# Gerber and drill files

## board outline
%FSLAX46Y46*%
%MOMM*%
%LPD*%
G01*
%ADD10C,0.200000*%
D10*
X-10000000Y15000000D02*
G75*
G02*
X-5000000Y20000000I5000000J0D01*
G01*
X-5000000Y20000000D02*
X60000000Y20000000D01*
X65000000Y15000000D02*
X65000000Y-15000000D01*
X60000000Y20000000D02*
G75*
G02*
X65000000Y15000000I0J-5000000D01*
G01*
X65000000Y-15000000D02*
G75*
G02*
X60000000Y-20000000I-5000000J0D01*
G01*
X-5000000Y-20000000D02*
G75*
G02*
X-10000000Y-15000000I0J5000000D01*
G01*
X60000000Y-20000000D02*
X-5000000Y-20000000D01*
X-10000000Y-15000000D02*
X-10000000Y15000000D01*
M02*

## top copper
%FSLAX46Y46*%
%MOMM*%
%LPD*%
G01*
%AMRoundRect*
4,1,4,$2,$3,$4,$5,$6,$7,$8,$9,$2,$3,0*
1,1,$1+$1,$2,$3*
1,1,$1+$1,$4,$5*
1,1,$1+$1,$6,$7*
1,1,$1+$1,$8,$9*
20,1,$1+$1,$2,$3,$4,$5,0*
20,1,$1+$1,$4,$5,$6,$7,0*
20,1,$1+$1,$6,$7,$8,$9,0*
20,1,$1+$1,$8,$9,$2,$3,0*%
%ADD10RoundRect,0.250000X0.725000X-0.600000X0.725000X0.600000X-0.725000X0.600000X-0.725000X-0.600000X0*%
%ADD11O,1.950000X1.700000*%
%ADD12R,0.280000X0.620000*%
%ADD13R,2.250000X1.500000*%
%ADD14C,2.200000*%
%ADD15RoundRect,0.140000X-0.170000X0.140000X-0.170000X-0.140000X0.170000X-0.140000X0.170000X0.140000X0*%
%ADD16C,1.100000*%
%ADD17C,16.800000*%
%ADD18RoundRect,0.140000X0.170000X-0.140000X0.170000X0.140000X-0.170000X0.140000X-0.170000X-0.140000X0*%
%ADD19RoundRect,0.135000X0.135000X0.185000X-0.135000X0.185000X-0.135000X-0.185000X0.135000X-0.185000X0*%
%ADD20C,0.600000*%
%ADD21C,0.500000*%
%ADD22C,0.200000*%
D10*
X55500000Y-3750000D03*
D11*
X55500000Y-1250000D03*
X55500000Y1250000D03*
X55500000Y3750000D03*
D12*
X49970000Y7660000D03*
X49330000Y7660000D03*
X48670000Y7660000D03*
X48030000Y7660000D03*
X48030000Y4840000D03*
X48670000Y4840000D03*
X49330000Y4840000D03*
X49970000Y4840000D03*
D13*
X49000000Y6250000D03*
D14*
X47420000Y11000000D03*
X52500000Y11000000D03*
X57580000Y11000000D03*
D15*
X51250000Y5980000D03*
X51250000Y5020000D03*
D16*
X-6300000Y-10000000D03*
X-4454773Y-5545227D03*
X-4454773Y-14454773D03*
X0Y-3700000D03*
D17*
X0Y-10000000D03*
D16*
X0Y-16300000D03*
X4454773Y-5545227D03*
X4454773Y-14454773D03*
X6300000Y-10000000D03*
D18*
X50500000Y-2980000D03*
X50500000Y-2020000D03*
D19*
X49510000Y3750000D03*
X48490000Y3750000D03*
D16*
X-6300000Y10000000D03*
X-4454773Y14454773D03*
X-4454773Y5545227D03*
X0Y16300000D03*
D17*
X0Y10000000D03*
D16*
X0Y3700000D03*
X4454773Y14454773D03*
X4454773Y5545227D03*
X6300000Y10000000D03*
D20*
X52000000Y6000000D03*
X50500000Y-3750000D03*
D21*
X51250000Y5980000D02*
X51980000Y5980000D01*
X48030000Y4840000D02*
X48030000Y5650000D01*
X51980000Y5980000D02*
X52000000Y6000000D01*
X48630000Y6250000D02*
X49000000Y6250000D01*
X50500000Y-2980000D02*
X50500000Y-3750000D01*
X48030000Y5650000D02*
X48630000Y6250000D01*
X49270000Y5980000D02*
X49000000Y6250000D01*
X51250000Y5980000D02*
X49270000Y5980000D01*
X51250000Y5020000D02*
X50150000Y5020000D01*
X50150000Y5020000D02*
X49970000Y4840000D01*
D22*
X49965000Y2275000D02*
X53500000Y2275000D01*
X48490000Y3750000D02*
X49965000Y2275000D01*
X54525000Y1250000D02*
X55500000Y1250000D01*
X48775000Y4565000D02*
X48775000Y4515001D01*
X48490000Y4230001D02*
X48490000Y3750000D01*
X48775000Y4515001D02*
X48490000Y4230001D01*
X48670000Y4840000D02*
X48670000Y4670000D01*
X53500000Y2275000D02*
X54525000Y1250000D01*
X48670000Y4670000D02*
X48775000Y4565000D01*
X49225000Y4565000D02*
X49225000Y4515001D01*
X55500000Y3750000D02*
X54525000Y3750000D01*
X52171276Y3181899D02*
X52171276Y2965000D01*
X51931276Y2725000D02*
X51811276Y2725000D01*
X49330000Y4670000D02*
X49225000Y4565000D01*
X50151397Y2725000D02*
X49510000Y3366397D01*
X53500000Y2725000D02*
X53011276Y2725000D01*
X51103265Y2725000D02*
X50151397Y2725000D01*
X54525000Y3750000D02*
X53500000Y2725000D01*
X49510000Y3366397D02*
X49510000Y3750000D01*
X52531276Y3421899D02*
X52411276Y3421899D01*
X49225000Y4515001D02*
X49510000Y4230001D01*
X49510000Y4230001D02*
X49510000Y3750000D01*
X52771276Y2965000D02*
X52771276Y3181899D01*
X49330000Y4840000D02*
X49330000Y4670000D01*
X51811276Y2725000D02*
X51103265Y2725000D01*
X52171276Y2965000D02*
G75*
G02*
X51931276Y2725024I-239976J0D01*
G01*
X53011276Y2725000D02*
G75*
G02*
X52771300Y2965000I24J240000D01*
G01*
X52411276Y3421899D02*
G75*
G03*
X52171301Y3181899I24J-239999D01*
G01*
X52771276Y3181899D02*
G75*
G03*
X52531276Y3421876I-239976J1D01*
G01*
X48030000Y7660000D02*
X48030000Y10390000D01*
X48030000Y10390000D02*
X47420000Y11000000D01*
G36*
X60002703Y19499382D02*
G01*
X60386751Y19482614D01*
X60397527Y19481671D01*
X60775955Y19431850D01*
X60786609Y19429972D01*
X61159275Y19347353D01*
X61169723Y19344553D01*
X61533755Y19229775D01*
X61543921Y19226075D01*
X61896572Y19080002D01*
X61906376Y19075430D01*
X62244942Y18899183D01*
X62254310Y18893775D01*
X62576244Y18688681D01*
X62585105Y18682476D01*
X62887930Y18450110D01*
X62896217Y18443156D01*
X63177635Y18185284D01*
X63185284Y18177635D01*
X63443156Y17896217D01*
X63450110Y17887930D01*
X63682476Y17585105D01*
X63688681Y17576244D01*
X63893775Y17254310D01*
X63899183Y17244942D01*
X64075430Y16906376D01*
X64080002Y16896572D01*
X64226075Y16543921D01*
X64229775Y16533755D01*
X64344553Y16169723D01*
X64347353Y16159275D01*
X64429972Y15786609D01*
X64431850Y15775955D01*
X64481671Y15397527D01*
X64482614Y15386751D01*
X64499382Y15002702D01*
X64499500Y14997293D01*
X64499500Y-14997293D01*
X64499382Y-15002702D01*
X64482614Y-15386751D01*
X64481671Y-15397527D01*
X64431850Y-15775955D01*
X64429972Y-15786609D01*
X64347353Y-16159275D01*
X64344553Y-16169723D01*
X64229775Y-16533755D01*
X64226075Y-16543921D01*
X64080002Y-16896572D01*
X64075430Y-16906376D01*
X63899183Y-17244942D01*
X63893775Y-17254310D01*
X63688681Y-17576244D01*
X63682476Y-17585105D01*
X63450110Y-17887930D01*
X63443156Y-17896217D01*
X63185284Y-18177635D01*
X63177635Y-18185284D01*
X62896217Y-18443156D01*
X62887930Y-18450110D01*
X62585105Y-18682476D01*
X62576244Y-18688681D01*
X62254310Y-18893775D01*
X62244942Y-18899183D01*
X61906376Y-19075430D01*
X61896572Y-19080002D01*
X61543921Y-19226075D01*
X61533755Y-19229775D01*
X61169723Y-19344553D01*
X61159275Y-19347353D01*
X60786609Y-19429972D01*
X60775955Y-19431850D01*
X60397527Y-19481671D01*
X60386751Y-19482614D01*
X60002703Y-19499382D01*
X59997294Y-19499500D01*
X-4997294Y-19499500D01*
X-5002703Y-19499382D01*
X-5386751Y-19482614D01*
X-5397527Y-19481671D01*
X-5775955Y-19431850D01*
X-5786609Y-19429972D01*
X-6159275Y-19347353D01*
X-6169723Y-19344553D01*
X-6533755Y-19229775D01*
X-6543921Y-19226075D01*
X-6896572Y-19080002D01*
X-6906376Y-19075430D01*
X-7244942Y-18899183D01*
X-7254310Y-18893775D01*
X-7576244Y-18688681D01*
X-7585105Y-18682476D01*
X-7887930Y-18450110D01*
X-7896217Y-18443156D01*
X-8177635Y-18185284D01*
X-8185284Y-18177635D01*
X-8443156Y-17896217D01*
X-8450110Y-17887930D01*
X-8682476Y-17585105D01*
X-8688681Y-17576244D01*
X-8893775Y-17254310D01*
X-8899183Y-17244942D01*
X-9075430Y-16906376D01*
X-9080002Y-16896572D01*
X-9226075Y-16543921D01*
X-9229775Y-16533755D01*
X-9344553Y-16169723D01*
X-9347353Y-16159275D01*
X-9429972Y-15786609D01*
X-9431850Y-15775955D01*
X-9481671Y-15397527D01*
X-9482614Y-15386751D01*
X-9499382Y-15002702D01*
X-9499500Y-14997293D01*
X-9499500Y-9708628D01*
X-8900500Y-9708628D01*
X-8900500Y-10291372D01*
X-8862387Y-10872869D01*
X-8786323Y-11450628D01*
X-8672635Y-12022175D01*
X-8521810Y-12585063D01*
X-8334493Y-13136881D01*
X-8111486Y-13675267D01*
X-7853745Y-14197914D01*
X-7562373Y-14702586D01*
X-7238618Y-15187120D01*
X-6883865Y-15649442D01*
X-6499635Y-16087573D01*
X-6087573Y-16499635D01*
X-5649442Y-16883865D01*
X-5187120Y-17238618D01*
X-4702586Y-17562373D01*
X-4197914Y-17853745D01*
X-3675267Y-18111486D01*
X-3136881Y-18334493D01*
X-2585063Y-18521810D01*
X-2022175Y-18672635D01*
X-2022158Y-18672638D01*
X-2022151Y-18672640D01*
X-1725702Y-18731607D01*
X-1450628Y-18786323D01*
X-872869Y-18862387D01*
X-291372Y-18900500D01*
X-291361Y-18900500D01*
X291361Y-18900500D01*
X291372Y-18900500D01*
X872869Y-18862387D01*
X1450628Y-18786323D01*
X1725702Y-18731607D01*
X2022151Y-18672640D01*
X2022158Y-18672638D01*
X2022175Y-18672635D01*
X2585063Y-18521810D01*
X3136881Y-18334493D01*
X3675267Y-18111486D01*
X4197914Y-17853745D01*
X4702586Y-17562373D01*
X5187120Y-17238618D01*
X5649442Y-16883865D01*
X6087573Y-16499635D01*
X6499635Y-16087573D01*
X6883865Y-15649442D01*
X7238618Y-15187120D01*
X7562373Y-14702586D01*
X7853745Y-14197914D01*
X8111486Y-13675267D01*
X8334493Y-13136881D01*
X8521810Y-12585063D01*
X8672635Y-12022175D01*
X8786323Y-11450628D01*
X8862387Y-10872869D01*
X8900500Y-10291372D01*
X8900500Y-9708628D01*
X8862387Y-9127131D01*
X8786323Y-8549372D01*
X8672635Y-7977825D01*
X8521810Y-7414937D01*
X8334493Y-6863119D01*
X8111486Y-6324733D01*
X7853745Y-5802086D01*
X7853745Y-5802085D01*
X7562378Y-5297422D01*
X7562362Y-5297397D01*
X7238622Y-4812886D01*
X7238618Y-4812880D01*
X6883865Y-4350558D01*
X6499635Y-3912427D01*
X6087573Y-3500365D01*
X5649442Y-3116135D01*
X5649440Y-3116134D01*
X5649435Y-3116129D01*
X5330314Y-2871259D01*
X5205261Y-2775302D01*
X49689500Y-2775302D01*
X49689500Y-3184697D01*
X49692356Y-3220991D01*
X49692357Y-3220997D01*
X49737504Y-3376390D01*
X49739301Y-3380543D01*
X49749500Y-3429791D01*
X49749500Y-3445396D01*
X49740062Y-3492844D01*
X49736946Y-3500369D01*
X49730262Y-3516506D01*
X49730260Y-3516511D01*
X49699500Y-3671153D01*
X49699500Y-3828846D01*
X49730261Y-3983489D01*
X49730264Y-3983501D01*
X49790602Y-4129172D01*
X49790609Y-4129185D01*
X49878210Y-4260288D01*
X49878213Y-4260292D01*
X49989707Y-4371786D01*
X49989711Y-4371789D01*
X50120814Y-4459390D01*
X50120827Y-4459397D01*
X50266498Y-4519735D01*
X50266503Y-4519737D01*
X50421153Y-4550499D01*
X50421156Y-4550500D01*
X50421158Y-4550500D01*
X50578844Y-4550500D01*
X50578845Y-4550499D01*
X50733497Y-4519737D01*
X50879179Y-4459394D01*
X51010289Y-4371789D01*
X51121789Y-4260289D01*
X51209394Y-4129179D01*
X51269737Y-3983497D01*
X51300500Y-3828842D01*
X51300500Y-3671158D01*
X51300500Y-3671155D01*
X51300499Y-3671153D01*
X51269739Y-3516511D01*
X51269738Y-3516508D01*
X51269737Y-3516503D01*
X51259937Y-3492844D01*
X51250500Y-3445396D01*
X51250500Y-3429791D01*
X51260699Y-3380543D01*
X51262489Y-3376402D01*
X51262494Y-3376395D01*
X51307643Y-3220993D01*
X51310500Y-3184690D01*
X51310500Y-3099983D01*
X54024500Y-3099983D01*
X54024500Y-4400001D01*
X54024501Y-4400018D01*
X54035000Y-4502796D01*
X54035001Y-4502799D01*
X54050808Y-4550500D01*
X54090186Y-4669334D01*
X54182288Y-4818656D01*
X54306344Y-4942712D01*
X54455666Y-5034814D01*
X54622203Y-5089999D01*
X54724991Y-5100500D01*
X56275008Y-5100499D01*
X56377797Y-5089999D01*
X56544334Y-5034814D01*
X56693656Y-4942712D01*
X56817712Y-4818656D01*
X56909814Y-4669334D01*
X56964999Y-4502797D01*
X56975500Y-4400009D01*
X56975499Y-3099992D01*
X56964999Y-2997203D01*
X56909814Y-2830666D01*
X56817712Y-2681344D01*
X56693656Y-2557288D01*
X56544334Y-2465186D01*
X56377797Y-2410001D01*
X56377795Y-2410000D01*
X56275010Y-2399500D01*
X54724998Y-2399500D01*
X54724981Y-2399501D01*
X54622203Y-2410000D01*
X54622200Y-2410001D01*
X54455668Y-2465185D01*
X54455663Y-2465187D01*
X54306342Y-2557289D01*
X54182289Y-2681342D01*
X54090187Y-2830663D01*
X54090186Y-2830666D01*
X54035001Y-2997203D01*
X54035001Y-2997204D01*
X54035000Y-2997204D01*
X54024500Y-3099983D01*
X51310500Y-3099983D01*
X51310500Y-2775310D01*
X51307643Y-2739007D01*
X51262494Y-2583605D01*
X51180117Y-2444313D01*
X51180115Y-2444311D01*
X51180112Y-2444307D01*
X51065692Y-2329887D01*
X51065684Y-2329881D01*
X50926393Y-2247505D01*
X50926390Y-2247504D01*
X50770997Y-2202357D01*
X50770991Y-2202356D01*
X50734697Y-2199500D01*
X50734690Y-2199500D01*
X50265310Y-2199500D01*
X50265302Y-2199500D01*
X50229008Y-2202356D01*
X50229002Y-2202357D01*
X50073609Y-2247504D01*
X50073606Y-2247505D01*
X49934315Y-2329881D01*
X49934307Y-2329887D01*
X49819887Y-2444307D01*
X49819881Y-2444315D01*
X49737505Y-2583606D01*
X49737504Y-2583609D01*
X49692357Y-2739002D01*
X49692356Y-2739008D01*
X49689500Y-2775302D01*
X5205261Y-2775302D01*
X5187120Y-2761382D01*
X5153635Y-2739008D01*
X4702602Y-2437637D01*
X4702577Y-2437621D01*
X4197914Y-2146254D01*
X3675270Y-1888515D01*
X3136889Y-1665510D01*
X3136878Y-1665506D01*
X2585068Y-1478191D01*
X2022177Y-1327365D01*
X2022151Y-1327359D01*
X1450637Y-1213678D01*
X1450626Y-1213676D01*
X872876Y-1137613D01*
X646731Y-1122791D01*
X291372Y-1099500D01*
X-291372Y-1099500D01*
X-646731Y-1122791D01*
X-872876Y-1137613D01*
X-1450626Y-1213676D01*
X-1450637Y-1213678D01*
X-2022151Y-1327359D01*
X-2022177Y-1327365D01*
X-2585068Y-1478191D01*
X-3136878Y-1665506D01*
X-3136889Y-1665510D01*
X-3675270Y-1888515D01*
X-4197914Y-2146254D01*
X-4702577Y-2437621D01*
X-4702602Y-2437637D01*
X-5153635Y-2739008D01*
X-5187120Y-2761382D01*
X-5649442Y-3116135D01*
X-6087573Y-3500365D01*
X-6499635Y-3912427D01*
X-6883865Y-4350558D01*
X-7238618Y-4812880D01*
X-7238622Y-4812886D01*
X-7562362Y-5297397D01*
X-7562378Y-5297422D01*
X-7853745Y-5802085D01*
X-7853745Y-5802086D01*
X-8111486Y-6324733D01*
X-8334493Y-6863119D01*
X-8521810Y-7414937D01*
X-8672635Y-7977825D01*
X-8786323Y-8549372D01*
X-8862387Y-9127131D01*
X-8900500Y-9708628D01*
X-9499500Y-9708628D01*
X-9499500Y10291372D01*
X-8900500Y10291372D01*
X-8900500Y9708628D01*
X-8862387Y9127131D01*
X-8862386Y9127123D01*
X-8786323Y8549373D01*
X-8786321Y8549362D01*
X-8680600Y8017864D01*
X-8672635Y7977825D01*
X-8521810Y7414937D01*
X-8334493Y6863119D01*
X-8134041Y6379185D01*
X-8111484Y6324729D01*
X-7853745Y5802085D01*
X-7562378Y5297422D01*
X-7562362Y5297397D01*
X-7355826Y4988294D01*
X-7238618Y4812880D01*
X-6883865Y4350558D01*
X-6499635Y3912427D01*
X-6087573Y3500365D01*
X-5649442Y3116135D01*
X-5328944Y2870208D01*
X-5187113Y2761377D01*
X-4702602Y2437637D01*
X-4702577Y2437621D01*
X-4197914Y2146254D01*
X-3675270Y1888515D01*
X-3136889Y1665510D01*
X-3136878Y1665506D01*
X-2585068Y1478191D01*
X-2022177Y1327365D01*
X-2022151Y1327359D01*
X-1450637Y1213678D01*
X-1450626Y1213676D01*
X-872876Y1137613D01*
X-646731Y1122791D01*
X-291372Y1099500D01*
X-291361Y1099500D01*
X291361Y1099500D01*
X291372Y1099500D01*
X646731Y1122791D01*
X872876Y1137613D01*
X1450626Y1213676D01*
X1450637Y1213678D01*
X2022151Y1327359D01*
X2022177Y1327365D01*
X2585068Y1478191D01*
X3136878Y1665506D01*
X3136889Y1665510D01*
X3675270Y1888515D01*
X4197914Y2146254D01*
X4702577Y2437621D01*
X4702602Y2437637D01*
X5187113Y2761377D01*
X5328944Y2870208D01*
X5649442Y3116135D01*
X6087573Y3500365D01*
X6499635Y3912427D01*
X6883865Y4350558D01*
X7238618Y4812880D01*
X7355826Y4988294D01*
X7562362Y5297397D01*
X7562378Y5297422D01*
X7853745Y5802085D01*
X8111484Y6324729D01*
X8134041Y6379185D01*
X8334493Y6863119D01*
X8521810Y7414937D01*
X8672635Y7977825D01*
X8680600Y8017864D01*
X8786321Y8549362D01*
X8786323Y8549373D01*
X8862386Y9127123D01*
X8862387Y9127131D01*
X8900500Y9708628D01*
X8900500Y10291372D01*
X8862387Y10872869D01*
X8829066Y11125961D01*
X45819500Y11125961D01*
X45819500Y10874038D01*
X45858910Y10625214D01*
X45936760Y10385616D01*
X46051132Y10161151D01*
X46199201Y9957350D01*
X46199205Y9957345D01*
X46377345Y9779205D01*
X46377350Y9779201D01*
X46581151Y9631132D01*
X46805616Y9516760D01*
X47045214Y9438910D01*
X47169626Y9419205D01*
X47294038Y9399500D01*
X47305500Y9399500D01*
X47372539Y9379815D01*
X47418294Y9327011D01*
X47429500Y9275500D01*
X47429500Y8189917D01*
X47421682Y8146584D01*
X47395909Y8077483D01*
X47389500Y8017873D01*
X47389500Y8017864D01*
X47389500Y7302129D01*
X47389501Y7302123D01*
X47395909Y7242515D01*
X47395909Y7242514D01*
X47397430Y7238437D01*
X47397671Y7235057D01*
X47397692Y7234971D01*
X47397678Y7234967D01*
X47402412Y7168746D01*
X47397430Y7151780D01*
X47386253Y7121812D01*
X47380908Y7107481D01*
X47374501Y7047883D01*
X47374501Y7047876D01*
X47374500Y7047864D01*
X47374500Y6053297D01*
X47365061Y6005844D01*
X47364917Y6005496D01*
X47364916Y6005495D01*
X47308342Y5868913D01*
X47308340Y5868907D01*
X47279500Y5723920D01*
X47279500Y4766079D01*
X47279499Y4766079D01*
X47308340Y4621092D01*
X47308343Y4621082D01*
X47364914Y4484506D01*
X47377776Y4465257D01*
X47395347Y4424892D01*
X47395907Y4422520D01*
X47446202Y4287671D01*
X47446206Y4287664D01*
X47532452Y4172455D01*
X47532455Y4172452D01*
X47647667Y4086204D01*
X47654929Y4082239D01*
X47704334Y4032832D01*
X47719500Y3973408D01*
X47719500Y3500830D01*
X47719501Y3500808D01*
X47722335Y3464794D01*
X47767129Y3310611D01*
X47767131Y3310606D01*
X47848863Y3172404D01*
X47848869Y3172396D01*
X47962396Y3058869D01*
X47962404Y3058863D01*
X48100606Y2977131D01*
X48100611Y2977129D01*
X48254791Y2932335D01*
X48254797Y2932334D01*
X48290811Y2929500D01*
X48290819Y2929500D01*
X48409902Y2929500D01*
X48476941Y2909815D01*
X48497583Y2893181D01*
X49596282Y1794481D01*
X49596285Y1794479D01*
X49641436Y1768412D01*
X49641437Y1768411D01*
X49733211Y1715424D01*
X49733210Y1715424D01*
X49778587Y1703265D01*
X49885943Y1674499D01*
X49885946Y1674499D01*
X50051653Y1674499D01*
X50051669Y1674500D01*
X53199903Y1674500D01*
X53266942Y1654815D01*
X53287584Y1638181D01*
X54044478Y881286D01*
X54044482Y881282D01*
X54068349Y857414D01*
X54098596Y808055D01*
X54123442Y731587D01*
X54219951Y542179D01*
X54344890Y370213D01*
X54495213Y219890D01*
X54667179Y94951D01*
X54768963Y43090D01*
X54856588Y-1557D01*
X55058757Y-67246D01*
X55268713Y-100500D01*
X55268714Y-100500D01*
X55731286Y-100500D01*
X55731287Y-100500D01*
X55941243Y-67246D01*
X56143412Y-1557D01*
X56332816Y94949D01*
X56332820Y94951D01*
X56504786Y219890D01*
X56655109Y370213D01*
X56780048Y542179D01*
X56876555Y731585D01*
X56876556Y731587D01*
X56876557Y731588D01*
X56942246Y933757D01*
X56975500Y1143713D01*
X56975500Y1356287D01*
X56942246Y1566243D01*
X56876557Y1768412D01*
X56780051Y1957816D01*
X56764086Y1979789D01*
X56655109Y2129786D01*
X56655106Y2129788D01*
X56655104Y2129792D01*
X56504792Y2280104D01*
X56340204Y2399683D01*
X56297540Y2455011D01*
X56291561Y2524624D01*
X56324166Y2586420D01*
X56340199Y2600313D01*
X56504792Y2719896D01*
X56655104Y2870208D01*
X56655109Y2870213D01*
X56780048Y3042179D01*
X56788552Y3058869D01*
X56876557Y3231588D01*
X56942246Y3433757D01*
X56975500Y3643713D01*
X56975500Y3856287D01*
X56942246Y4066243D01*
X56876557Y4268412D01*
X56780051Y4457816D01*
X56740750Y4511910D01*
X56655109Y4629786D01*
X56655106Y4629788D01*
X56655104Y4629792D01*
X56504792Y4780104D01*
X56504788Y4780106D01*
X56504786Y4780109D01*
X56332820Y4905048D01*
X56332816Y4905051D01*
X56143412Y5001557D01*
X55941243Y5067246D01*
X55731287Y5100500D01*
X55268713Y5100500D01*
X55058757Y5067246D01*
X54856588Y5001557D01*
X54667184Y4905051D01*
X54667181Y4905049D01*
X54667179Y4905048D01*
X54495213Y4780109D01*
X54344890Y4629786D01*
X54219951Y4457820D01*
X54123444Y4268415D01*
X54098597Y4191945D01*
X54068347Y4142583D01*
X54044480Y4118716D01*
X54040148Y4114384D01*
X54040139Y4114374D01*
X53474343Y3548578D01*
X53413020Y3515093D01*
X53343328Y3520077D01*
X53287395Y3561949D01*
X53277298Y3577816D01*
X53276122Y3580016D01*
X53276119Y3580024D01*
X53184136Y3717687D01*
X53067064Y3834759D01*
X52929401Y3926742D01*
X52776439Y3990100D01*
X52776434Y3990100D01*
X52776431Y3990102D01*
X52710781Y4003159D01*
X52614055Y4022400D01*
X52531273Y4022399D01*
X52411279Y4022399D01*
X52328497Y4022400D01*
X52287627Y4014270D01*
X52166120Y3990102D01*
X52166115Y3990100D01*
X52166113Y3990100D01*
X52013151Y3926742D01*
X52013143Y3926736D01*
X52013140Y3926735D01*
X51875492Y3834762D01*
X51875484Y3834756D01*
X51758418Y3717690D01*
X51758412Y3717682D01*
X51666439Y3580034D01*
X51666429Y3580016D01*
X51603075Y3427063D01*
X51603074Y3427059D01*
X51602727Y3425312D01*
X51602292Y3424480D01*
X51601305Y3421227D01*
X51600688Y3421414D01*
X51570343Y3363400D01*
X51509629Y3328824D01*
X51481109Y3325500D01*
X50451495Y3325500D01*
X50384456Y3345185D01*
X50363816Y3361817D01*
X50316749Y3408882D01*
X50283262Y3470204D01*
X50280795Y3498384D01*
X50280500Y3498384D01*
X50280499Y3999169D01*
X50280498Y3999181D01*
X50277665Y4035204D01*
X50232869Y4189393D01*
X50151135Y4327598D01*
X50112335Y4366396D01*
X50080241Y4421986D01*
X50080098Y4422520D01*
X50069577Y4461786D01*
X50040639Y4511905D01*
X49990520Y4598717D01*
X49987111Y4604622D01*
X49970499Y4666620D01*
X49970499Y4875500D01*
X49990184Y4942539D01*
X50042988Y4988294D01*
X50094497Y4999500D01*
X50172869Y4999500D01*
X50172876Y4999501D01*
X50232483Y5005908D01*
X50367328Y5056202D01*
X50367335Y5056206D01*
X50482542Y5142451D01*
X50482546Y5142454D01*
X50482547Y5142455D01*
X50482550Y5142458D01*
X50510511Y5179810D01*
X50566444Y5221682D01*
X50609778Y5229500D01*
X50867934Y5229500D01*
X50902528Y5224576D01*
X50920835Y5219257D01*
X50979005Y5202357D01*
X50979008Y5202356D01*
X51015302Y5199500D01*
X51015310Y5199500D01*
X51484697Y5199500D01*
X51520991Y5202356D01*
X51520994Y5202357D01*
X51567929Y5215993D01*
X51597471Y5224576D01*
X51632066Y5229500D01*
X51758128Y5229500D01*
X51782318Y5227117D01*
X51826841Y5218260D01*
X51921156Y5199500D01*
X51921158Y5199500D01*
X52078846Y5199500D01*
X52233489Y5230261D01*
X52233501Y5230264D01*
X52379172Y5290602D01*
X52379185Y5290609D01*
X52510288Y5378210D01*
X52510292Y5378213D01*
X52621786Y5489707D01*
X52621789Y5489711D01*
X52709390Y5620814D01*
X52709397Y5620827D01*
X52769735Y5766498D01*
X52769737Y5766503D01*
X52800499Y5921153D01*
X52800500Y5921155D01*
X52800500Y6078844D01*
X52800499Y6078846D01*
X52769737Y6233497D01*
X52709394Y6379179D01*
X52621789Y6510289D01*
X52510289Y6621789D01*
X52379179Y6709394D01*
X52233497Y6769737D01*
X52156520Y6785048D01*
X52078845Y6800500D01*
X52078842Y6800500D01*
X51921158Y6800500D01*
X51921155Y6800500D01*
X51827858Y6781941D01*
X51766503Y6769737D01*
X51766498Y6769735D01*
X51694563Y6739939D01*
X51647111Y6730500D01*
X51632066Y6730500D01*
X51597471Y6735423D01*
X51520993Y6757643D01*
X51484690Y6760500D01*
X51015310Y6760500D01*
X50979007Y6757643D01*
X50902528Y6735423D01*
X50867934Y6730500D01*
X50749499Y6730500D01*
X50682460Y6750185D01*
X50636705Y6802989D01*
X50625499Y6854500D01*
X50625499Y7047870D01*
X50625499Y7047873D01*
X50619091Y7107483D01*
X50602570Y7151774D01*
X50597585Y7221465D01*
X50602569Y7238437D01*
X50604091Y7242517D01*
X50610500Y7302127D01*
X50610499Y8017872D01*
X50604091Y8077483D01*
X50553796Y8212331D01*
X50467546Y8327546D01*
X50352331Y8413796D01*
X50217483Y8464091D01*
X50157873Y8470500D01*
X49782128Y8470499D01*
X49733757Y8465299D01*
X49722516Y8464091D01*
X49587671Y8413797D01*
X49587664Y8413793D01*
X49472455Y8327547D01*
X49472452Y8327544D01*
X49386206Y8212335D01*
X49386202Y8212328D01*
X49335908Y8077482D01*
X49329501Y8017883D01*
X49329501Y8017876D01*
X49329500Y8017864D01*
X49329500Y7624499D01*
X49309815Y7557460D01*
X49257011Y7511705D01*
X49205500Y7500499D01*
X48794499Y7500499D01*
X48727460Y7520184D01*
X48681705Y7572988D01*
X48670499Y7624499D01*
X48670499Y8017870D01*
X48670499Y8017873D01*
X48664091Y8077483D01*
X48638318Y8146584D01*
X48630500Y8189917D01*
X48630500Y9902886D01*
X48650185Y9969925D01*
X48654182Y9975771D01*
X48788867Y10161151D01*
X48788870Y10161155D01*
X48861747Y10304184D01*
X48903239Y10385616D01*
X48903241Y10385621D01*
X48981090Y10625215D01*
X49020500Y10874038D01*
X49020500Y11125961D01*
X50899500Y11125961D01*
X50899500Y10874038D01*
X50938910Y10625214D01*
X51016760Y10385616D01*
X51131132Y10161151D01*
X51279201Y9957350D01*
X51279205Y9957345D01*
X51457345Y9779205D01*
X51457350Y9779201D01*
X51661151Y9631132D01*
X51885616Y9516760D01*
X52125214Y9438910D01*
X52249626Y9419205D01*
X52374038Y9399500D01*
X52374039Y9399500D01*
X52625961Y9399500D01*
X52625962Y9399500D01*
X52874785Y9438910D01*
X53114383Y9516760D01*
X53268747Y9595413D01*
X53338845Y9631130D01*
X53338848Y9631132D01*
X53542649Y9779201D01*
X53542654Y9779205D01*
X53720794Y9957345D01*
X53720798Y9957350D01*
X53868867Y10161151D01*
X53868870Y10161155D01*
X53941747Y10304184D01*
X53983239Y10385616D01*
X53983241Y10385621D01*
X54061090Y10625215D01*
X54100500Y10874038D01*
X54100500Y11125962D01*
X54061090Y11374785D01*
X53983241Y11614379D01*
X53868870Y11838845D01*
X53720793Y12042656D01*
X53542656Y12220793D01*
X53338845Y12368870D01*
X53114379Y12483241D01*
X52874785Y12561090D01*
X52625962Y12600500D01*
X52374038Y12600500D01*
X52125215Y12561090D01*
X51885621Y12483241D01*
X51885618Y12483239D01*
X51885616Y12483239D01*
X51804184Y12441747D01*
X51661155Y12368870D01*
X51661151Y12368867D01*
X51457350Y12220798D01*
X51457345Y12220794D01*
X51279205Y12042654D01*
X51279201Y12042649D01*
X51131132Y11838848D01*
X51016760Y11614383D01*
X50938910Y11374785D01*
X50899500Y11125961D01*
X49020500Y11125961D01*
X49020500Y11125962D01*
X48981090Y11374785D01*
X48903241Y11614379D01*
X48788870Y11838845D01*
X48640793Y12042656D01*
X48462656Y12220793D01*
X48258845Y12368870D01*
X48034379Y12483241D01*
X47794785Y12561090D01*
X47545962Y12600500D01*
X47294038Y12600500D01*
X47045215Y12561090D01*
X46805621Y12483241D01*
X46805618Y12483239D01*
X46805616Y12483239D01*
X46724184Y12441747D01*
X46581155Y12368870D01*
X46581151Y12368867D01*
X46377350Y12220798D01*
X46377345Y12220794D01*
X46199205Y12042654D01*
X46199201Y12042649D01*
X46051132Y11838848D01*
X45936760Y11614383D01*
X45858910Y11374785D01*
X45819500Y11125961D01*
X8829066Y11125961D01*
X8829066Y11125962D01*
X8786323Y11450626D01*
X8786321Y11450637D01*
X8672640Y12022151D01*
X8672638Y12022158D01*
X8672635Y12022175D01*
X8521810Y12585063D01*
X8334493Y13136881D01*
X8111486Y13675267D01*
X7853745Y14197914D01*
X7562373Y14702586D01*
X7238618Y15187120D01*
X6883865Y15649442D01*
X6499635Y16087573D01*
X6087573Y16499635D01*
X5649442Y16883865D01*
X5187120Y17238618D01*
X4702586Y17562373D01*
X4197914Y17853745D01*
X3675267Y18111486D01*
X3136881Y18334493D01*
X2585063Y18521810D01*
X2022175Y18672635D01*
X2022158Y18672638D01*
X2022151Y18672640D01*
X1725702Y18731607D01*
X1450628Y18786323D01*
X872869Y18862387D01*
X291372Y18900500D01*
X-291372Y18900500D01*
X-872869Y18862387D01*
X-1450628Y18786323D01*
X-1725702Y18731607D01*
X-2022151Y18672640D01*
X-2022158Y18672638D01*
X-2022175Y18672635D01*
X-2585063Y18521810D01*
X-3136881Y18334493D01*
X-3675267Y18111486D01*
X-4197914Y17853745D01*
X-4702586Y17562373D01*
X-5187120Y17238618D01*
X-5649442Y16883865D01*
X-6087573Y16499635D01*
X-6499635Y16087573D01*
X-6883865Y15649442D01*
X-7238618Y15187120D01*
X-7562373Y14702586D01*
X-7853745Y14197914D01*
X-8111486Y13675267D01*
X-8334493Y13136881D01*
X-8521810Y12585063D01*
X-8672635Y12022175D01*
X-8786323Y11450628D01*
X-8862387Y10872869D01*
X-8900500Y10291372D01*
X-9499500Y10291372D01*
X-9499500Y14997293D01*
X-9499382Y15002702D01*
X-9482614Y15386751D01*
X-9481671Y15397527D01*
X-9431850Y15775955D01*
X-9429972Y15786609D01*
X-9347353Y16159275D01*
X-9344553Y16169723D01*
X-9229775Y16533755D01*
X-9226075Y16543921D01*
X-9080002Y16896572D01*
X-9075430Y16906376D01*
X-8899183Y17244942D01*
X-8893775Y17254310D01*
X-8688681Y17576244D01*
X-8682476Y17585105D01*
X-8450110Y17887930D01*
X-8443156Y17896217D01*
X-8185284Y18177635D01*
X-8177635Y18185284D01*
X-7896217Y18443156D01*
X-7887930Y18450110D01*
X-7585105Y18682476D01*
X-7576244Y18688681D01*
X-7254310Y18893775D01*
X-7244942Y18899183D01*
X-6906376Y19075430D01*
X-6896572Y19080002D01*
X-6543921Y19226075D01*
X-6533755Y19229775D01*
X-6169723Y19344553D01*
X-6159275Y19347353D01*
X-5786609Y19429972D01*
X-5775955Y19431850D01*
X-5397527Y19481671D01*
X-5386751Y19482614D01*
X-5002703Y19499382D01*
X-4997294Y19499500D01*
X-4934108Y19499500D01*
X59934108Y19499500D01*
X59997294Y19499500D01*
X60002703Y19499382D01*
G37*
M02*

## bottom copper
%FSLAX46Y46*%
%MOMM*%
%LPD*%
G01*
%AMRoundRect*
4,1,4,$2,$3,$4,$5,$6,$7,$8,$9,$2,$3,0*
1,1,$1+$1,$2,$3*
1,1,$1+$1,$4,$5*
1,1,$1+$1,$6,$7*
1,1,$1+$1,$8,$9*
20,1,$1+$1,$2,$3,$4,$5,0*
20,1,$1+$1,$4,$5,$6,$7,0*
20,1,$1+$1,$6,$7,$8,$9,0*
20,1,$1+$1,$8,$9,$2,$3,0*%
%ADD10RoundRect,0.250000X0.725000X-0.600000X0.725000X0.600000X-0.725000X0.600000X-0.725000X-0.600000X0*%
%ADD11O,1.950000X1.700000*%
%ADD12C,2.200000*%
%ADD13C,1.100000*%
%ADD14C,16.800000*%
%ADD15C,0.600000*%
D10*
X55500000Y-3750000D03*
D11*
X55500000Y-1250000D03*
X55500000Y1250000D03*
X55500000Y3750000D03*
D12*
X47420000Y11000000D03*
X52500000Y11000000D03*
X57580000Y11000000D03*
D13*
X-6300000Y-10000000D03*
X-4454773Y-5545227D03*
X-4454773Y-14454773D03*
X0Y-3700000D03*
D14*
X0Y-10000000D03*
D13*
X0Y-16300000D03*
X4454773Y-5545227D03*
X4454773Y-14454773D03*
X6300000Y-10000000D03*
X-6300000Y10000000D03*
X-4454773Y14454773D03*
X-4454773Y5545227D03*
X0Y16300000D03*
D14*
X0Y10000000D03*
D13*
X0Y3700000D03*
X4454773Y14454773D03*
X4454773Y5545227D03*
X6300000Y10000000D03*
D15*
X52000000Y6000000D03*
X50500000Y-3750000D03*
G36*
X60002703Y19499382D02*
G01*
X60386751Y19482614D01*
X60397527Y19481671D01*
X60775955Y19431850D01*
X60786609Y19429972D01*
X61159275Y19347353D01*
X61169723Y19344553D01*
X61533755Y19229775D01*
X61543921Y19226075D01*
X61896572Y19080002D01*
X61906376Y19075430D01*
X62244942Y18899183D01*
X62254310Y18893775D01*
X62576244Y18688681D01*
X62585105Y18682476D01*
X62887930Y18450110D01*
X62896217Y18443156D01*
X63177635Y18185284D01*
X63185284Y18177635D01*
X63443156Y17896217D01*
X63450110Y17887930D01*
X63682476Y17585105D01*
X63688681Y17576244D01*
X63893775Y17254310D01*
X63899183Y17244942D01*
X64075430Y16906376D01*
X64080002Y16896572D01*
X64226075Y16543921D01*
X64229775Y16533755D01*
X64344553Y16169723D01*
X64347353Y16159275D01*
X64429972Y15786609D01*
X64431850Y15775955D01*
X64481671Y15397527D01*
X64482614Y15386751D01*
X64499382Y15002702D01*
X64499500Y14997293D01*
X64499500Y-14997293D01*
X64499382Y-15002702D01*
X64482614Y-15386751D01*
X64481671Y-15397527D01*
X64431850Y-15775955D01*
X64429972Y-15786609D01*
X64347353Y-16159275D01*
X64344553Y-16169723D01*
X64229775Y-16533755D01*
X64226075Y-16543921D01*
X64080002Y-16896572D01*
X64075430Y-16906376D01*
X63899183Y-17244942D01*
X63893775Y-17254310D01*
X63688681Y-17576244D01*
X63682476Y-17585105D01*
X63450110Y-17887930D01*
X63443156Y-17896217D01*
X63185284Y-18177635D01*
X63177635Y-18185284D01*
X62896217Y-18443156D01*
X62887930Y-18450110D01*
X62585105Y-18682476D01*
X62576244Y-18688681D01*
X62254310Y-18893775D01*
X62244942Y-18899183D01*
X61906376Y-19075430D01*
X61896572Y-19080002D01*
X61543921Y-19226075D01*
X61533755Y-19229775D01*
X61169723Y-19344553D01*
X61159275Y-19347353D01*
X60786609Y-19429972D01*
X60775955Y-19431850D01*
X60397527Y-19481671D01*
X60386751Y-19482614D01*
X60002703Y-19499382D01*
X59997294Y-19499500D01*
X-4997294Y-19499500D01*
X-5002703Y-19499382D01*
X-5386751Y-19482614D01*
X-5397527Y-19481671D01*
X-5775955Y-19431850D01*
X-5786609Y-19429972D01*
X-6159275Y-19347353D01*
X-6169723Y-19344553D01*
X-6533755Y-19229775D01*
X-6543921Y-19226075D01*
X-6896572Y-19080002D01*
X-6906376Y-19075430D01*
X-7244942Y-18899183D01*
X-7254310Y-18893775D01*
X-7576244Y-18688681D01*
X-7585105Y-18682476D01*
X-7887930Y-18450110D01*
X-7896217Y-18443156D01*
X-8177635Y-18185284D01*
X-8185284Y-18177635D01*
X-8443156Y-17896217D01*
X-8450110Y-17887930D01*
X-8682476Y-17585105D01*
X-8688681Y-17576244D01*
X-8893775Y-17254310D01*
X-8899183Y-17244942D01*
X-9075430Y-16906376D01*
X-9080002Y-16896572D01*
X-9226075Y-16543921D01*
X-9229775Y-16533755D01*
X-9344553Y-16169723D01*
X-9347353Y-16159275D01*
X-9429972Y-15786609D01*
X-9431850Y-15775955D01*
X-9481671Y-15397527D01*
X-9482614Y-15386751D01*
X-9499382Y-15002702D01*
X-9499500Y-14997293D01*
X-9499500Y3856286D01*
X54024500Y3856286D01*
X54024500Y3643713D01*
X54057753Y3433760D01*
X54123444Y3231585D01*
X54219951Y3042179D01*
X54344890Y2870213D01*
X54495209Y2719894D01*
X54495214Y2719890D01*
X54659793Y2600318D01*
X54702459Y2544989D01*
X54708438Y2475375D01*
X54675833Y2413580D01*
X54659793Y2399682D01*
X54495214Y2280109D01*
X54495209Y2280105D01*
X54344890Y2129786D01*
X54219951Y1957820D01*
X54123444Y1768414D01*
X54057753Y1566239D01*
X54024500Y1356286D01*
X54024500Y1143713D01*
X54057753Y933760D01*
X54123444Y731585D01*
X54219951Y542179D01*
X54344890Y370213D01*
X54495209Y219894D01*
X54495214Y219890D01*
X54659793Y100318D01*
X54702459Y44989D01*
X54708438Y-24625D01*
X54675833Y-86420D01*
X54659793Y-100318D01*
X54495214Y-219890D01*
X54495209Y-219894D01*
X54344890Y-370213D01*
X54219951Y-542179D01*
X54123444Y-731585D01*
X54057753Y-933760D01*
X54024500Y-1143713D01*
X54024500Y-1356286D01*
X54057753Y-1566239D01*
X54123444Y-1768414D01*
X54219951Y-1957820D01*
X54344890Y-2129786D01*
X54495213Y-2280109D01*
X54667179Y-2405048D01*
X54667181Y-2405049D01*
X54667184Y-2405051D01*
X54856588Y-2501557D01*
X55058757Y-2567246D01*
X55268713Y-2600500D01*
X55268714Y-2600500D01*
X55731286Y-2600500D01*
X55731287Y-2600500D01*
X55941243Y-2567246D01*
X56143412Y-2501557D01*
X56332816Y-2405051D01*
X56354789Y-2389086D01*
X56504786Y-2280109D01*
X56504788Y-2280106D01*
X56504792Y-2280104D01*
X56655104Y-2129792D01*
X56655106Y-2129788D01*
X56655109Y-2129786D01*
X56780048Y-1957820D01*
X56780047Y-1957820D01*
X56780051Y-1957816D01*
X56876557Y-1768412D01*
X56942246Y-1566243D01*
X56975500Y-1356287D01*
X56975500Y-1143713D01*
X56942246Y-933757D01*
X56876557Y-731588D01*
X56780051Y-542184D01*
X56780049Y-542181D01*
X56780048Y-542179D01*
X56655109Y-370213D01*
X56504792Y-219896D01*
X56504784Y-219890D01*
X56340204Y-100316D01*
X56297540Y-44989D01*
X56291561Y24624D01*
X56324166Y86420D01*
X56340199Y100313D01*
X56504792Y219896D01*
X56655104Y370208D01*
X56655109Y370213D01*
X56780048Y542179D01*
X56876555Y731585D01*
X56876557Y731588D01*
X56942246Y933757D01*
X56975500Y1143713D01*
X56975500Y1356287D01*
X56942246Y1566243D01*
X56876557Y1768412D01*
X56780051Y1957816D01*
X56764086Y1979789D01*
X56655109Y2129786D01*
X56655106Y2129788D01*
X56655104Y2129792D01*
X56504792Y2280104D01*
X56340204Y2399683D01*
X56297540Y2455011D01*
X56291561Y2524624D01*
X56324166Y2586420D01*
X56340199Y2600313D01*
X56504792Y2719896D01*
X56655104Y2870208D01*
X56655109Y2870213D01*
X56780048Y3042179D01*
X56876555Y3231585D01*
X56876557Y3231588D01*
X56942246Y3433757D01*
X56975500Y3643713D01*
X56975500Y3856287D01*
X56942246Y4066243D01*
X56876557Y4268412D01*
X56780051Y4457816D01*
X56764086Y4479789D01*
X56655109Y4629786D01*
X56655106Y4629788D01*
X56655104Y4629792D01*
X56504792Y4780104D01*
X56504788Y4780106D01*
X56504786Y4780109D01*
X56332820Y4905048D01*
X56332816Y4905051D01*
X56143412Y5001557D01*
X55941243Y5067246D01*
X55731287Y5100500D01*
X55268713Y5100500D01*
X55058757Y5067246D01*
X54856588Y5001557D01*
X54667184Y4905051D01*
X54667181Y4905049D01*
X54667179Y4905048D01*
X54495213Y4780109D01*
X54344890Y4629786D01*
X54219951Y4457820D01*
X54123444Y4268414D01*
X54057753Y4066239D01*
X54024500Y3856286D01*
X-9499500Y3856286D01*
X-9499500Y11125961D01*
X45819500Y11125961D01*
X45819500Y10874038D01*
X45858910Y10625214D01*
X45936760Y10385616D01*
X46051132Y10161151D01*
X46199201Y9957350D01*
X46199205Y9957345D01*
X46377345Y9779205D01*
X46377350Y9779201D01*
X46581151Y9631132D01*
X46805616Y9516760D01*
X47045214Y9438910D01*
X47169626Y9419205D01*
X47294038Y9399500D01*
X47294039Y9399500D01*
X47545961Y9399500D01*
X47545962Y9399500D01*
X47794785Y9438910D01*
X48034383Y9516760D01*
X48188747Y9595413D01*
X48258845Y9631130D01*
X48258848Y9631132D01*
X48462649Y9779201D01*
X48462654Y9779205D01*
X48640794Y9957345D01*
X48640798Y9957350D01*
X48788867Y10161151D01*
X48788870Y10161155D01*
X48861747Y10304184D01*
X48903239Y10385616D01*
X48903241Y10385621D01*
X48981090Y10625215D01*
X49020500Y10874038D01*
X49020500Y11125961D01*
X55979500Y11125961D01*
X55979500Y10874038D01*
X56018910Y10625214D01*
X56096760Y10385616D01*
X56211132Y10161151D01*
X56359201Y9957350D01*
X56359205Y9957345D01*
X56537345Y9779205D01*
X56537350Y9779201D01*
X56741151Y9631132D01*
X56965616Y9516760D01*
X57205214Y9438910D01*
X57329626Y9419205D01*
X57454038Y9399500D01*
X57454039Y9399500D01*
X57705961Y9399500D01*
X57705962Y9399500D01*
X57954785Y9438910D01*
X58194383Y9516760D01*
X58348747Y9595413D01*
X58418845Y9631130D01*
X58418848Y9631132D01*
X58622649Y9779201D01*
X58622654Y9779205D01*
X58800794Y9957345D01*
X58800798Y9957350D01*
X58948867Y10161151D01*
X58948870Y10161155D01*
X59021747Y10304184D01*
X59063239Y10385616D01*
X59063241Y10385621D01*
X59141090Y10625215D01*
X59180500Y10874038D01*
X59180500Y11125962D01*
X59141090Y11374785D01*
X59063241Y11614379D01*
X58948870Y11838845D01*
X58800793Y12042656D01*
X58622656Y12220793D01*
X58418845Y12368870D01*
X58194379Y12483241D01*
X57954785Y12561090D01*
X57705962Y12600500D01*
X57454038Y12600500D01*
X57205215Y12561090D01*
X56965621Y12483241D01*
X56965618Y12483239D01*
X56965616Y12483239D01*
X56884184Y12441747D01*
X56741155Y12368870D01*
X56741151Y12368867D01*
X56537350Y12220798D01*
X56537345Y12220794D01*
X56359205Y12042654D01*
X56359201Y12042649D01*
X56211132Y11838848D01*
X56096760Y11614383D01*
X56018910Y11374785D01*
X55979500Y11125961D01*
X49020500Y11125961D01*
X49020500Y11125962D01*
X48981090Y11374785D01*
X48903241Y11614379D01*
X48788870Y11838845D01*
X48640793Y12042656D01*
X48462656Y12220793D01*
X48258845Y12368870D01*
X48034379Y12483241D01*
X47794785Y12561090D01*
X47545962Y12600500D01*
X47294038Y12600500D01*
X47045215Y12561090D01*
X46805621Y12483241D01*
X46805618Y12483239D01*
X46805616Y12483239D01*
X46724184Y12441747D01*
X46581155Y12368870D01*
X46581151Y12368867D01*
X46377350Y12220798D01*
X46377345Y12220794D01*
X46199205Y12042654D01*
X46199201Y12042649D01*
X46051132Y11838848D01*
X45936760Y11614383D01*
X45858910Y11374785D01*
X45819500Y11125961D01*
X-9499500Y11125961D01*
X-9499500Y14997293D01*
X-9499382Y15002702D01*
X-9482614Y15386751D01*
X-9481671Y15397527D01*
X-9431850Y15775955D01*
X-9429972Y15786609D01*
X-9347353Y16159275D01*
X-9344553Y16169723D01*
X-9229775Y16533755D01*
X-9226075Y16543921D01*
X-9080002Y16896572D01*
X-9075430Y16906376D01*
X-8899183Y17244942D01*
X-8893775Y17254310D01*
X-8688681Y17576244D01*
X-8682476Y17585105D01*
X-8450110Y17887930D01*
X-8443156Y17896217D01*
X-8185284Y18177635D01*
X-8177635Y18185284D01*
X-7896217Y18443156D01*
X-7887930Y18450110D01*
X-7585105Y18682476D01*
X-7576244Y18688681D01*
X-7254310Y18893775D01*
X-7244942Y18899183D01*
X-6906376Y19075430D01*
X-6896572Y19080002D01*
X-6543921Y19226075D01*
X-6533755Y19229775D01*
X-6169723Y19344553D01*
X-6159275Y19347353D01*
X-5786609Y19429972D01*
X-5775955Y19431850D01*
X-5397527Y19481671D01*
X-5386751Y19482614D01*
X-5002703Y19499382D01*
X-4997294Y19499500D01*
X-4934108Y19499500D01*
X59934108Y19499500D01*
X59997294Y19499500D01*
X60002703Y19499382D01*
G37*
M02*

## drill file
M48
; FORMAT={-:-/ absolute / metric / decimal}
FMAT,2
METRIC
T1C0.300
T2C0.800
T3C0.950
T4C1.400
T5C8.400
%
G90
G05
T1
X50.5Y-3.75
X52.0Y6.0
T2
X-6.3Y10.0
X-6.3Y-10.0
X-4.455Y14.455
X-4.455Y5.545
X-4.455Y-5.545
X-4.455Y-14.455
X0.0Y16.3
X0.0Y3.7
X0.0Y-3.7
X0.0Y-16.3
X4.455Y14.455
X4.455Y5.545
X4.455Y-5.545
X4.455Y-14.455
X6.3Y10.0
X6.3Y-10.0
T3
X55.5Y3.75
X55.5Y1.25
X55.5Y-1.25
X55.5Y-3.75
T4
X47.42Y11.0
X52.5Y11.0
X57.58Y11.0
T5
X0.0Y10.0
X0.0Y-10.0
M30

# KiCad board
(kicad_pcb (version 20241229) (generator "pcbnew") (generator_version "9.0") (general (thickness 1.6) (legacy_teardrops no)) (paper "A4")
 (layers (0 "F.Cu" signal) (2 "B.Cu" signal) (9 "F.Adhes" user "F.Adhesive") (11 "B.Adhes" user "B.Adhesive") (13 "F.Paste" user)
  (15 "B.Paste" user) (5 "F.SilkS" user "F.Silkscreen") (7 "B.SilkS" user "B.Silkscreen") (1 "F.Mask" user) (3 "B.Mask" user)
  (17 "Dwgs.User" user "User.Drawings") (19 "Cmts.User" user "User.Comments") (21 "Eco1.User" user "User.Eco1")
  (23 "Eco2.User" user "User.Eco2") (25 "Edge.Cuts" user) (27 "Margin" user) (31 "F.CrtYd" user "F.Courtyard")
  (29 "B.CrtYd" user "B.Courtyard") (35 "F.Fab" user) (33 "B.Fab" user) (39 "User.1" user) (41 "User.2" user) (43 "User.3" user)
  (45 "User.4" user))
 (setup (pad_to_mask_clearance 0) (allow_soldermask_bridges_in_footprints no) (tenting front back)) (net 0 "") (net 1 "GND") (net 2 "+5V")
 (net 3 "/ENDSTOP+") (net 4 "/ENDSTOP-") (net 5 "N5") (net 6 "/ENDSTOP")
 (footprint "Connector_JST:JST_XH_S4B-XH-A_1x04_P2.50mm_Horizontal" (layer "F.Cu") (at 55.5 3.75 90)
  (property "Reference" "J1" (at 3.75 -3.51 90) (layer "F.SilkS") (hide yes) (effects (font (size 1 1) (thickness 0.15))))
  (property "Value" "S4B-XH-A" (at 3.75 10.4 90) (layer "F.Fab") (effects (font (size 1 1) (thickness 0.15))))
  (pad "1" thru_hole roundrect (at 0 0 90) (size 1.7 1.95) (drill 0.95) (layers "*.Cu" "*.Mask") (remove_unused_layers no)
   (roundrect_rratio 0.147059) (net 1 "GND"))
  (pad "2" thru_hole oval (at 2.5 0 90) (size 1.7 1.95) (drill 0.95) (layers "*.Cu" "*.Mask") (remove_unused_layers no) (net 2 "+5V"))
  (pad "3" thru_hole oval (at 5 0 90) (size 1.7 1.95) (drill 0.95) (layers "*.Cu" "*.Mask") (remove_unused_layers no) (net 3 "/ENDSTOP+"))
  (pad "4" thru_hole oval (at 7.5 0 90) (size 1.7 1.95) (drill 0.95) (layers "*.Cu" "*.Mask") (remove_unused_layers no) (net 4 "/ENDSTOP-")))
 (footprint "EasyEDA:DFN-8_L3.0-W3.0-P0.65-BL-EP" (layer "F.Cu") (at 49 -6.25 180)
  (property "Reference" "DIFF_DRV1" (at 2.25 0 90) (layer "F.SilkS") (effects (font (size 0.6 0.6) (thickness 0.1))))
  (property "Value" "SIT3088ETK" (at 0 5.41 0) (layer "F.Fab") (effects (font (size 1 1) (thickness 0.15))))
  (pad "1" smd rect (at -0.97 1.41 180) (size 0.28 0.62) (layers "F.Cu" "F.Mask" "F.Paste") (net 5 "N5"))
  (pad "2" smd rect (at -0.33 1.41 180) (size 0.28 0.62) (layers "F.Cu" "F.Mask" "F.Paste") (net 2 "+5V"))
  (pad "3" smd rect (at 0.33 1.41 180) (size 0.28 0.62) (layers "F.Cu" "F.Mask" "F.Paste") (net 2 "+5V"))
  (pad "4" smd rect (at 0.97 1.41 180) (size 0.28 0.62) (layers "F.Cu" "F.Mask" "F.Paste") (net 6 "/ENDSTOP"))
  (pad "5" smd rect (at 0.97 -1.41 180) (size 0.28 0.62) (layers "F.Cu" "F.Mask" "F.Paste") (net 1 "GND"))
  (pad "6" smd rect (at 0.33 -1.41 180) (size 0.28 0.62) (layers "F.Cu" "F.Mask" "F.Paste") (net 3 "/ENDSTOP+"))
  (pad "7" smd rect (at -0.33 -1.41 180) (size 0.28 0.62) (layers "F.Cu" "F.Mask" "F.Paste") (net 4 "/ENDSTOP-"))
  (pad "8" smd rect (at -0.97 -1.41 180) (size 0.28 0.62) (layers "F.Cu" "F.Mask" "F.Paste") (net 2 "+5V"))
  (pad "9" smd rect (at 0 0 180) (size 2.25 1.5) (layers "F.Cu" "F.Mask" "F.Paste") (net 1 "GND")))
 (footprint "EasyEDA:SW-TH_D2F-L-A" (layer "F.Cu") (at 52.5 -11)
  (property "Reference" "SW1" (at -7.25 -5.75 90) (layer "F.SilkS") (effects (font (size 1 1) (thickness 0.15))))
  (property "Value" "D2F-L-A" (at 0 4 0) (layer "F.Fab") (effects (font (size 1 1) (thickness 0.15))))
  (pad "1" thru_hole circle (at -5.08 0) (size 2.2 2.2) (drill 1.399997) (layers "*.Cu" "*.Mask") (remove_unused_layers no)
   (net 6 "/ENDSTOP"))
  (pad "2" thru_hole circle (at 0 0) (size 2.2 2.2) (drill 1.399997) (layers "*.Cu" "*.Mask") (remove_unused_layers no) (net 1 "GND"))
  (pad "3" thru_hole circle (at 5.08 0) (size 2.2 2.2) (drill 1.399997) (layers "*.Cu" "*.Mask") (remove_unused_layers no) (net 2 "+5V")))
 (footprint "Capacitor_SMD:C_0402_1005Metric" (layer "F.Cu") (at 51.25 -5.5 -90)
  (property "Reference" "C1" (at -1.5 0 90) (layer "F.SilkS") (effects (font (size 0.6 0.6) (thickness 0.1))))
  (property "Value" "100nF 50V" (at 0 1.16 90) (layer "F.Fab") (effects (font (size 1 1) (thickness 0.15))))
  (pad "1" smd roundrect (at -0.48 0 270) (size 0.56 0.62) (layers "F.Cu" "F.Mask" "F.Paste") (roundrect_rratio 0.25) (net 1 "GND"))
  (pad "2" smd roundrect (at 0.48 0 270) (size 0.56 0.62) (layers "F.Cu" "F.Mask" "F.Paste") (roundrect_rratio 0.25) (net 2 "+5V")))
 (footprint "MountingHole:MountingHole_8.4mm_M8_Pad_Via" (layer "F.Cu") (at 0 10)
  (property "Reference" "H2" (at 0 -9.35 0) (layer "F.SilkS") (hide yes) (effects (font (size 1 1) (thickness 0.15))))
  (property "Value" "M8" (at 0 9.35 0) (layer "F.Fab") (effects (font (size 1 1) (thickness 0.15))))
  (pad "1" thru_hole circle (at -6.3 0) (size 1.1 1.1) (drill 0.8) (layers "*.Cu" "*.Mask") (remove_unused_layers no) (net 1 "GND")
   (zone_connect 2))
  (pad "1" thru_hole circle (at -4.454773 -4.454773) (size 1.1 1.1) (drill 0.8) (layers "*.Cu" "*.Mask") (remove_unused_layers no)
   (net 1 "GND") (zone_connect 2))
  (pad "1" thru_hole circle (at -4.454773 4.454773) (size 1.1 1.1) (drill 0.8) (layers "*.Cu" "*.Mask") (remove_unused_layers no)
   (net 1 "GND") (zone_connect 2))
  (pad "1" thru_hole circle (at 0 -6.3) (size 1.1 1.1) (drill 0.8) (layers "*.Cu" "*.Mask") (remove_unused_layers no) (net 1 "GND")
   (zone_connect 2))
  (pad "1" thru_hole circle (at 0 0) (size 16.8 16.8) (drill 8.4) (layers "*.Cu" "*.Mask") (remove_unused_layers no) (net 1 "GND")
   (zone_connect 2))
  (pad "1" thru_hole circle (at 0 6.3) (size 1.1 1.1) (drill 0.8) (layers "*.Cu" "*.Mask") (remove_unused_layers no) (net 1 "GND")
   (zone_connect 2))
  (pad "1" thru_hole circle (at 4.454773 -4.454773) (size 1.1 1.1) (drill 0.8) (layers "*.Cu" "*.Mask") (remove_unused_layers no)
   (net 1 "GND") (zone_connect 2))
  (pad "1" thru_hole circle (at 4.454773 4.454773) (size 1.1 1.1) (drill 0.8) (layers "*.Cu" "*.Mask") (remove_unused_layers no)
   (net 1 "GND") (zone_connect 2))
  (pad "1" thru_hole circle (at 6.3 0) (size 1.1 1.1) (drill 0.8) (layers "*.Cu" "*.Mask") (remove_unused_layers no) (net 1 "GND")
   (zone_connect 2)))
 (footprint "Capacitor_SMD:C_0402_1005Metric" (layer "F.Cu") (at 50.5 2.5 90)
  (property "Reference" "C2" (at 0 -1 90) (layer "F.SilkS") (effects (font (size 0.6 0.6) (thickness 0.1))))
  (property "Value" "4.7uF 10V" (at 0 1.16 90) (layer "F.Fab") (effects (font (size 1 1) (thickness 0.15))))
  (pad "1" smd roundrect (at -0.48 0 90) (size 0.56 0.62) (layers "F.Cu" "F.Mask" "F.Paste") (roundrect_rratio 0.25) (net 1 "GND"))
  (pad "2" smd roundrect (at 0.48 0 90) (size 0.56 0.62) (layers "F.Cu" "F.Mask" "F.Paste") (roundrect_rratio 0.25) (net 2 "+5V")))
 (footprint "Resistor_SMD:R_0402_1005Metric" (layer "F.Cu") (at 49 -3.75 180)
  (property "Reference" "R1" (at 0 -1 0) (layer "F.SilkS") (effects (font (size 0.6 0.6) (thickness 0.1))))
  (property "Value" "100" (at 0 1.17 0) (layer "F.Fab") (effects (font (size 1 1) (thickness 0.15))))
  (pad "1" smd roundrect (at -0.51 0 180) (size 0.54 0.64) (layers "F.Cu" "F.Mask" "F.Paste") (roundrect_rratio 0.25) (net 4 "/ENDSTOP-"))
  (pad "2" smd roundrect (at 0.51 0 180) (size 0.54 0.64) (layers "F.Cu" "F.Mask" "F.Paste") (roundrect_rratio 0.25) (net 3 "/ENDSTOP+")))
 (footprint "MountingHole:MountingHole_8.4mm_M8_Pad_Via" (layer "F.Cu") (at 0 -10)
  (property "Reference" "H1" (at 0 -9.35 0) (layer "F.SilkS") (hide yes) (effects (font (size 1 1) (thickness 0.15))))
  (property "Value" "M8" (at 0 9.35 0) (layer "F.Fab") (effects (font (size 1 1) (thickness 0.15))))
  (pad "1" thru_hole circle (at -6.3 0) (size 1.1 1.1) (drill 0.8) (layers "*.Cu" "*.Mask") (remove_unused_layers no) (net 1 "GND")
   (zone_connect 2))
  (pad "1" thru_hole circle (at -4.454773 -4.454773) (size 1.1 1.1) (drill 0.8) (layers "*.Cu" "*.Mask") (remove_unused_layers no)
   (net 1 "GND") (zone_connect 2))
  (pad "1" thru_hole circle (at -4.454773 4.454773) (size 1.1 1.1) (drill 0.8) (layers "*.Cu" "*.Mask") (remove_unused_layers no)
   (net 1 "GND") (zone_connect 2))
  (pad "1" thru_hole circle (at 0 -6.3) (size 1.1 1.1) (drill 0.8) (layers "*.Cu" "*.Mask") (remove_unused_layers no) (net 1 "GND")
   (zone_connect 2))
  (pad "1" thru_hole circle (at 0 0) (size 16.8 16.8) (drill 8.4) (layers "*.Cu" "*.Mask") (remove_unused_layers no) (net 1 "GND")
   (zone_connect 2))
  (pad "1" thru_hole circle (at 0 6.3) (size 1.1 1.1) (drill 0.8) (layers "*.Cu" "*.Mask") (remove_unused_layers no) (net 1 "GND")
   (zone_connect 2))
  (pad "1" thru_hole circle (at 4.454773 -4.454773) (size 1.1 1.1) (drill 0.8) (layers "*.Cu" "*.Mask") (remove_unused_layers no)
   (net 1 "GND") (zone_connect 2))
  (pad "1" thru_hole circle (at 4.454773 4.454773) (size 1.1 1.1) (drill 0.8) (layers "*.Cu" "*.Mask") (remove_unused_layers no)
   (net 1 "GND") (zone_connect 2))
  (pad "1" thru_hole circle (at 6.3 0) (size 1.1 1.1) (drill 0.8) (layers "*.Cu" "*.Mask") (remove_unused_layers no) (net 1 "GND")
   (zone_connect 2)))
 (gr_arc (start -10 -15) (mid -8.535534 -18.535534) (end -5 -20) (stroke (width 0.2) (type default)) (layer "Edge.Cuts"))
 (gr_line (start -5 -20) (end 60 -20) (stroke (width 0.2) (type default)) (layer "Edge.Cuts"))
 (gr_line (start 65 -15) (end 65 15) (stroke (width 0.2) (type default)) (layer "Edge.Cuts"))
 (gr_arc (start 60 -20) (mid 63.535534 -18.535534) (end 65 -15) (stroke (width 0.2) (type default)) (layer "Edge.Cuts"))
 (gr_arc (start 65 15) (mid 63.535534 18.535534) (end 60 20) (stroke (width 0.2) (type default)) (layer "Edge.Cuts"))
 (gr_arc (start -5 20) (mid -8.535534 18.535534) (end -10 15) (stroke (width 0.2) (type default)) (layer "Edge.Cuts"))
 (gr_line (start 60 20) (end -5 20) (stroke (width 0.2) (type default)) (layer "Edge.Cuts"))
 (gr_line (start -10 15) (end -10 -15) (stroke (width 0.2) (type default)) (layer "Edge.Cuts"))
 (segment (start 51.25 -5.98) (end 51.98 -5.98) (width 0.5) (layer "F.Cu") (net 1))
 (segment (start 48.03 -4.84) (end 48.03 -5.65) (width 0.5) (layer "F.Cu") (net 1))
 (segment (start 51.98 -5.98) (end 52 -6) (width 0.5) (layer "F.Cu") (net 1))
 (segment (start 48.63 -6.25) (end 49 -6.25) (width 0.5) (layer "F.Cu") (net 1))
 (segment (start 50.5 2.98) (end 50.5 3.75) (width 0.5) (layer "F.Cu") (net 1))
 (segment (start 48.03 -5.65) (end 48.63 -6.25) (width 0.5) (layer "F.Cu") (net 1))
 (segment (start 49.27 -5.98) (end 49 -6.25) (width 0.5) (layer "F.Cu") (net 1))
 (segment (start 51.25 -5.98) (end 49.27 -5.98) (width 0.5) (layer "F.Cu") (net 1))
 (via (at 52 -6) (size 0.6) (drill 0.3) (layers "F.Cu" "B.Cu") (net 1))
 (via (at 50.5 3.75) (size 0.6) (drill 0.3) (layers "F.Cu" "B.Cu") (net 1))
 (segment (start 51.25 -5.02) (end 50.15 -5.02) (width 0.5) (layer "F.Cu") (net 2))
 (segment (start 50.15 -5.02) (end 49.97 -4.84) (width 0.5) (layer "F.Cu") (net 2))
 (segment (start 49.965 -2.275) (end 53.5 -2.275) (width 0.2) (layer "F.Cu") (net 3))
 (segment (start 48.49 -3.75) (end 49.965 -2.275) (width 0.2) (layer "F.Cu") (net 3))
 (segment (start 54.525 -1.25) (end 55.5 -1.25) (width 0.2) (layer "F.Cu") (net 3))
 (segment (start 48.775 -4.565) (end 48.775 -4.515001) (width 0.2) (layer "F.Cu") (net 3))
 (segment (start 48.49 -4.230001) (end 48.49 -3.75) (width 0.2) (layer "F.Cu") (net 3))
 (segment (start 48.775 -4.515001) (end 48.49 -4.230001) (width 0.2) (layer "F.Cu") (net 3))
 (segment (start 48.67 -4.84) (end 48.67 -4.67) (width 0.2) (layer "F.Cu") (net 3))
 (segment (start 53.5 -2.275) (end 54.525 -1.25) (width 0.2) (layer "F.Cu") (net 3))
 (segment (start 48.67 -4.67) (end 48.775 -4.565) (width 0.2) (layer "F.Cu") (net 3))
 (segment (start 49.225 -4.565) (end 49.225 -4.515001) (width 0.2) (layer "F.Cu") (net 4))
 (segment (start 55.5 -3.75) (end 54.525 -3.75) (width 0.2) (layer "F.Cu") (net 4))
 (segment (start 52.171276 -3.181899) (end 52.171276 -2.965) (width 0.2) (layer "F.Cu") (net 4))
 (segment (start 51.931276 -2.725) (end 51.811276 -2.725) (width 0.2) (layer "F.Cu") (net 4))
 (segment (start 49.33 -4.67) (end 49.225 -4.565) (width 0.2) (layer "F.Cu") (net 4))
 (segment (start 50.151397 -2.725) (end 49.51 -3.366397) (width 0.2) (layer "F.Cu") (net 4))
 (segment (start 53.5 -2.725) (end 53.011276 -2.725) (width 0.2) (layer "F.Cu") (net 4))
 (segment (start 51.103265 -2.725) (end 50.151397 -2.725) (width 0.2) (layer "F.Cu") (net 4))
 (segment (start 54.525 -3.75) (end 53.5 -2.725) (width 0.2) (layer "F.Cu") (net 4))
 (segment (start 49.51 -3.366397) (end 49.51 -3.75) (width 0.2) (layer "F.Cu") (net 4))
 (segment (start 52.531276 -3.421899) (end 52.411276 -3.421899) (width 0.2) (layer "F.Cu") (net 4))
 (segment (start 49.225 -4.515001) (end 49.51 -4.230001) (width 0.2) (layer "F.Cu") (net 4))
 (segment (start 49.51 -4.230001) (end 49.51 -3.75) (width 0.2) (layer "F.Cu") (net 4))
 (segment (start 52.771276 -2.965) (end 52.771276 -3.181899) (width 0.2) (layer "F.Cu") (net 4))
 (segment (start 49.33 -4.84) (end 49.33 -4.67) (width 0.2) (layer "F.Cu") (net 4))
 (segment (start 51.811276 -2.725) (end 51.103265 -2.725) (width 0.2) (layer "F.Cu") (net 4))
 (arc (start 52.171276 -2.965) (mid 52.100982 -2.795294) (end 51.931276 -2.725) (width 0.2) (layer "F.Cu") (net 4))
 (arc (start 53.011276 -2.725) (mid 52.84157 -2.795294) (end 52.771276 -2.965) (width 0.2) (layer "F.Cu") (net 4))
 (arc (start 52.411276 -3.421899) (mid 52.24157 -3.351605) (end 52.171276 -3.181899) (width 0.2) (layer "F.Cu") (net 4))
 (arc (start 52.771276 -3.181899) (mid 52.700982 -3.351605) (end 52.531276 -3.421899) (width 0.2) (layer "F.Cu") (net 4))
 (segment (start 48.03 -7.66) (end 48.03 -10.39) (width 0.2) (layer "F.Cu") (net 6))
 (segment (start 48.03 -10.39) (end 47.42 -11) (width 0.2) (layer "F.Cu") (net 6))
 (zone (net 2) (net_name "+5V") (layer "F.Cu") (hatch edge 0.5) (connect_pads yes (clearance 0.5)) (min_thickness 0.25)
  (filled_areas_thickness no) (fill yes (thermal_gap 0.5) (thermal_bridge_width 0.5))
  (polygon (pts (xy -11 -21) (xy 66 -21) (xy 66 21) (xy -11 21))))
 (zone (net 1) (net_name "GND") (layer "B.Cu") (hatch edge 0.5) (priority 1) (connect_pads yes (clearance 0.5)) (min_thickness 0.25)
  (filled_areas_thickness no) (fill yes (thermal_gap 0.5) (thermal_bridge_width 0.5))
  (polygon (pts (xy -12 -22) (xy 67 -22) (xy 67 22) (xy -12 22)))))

